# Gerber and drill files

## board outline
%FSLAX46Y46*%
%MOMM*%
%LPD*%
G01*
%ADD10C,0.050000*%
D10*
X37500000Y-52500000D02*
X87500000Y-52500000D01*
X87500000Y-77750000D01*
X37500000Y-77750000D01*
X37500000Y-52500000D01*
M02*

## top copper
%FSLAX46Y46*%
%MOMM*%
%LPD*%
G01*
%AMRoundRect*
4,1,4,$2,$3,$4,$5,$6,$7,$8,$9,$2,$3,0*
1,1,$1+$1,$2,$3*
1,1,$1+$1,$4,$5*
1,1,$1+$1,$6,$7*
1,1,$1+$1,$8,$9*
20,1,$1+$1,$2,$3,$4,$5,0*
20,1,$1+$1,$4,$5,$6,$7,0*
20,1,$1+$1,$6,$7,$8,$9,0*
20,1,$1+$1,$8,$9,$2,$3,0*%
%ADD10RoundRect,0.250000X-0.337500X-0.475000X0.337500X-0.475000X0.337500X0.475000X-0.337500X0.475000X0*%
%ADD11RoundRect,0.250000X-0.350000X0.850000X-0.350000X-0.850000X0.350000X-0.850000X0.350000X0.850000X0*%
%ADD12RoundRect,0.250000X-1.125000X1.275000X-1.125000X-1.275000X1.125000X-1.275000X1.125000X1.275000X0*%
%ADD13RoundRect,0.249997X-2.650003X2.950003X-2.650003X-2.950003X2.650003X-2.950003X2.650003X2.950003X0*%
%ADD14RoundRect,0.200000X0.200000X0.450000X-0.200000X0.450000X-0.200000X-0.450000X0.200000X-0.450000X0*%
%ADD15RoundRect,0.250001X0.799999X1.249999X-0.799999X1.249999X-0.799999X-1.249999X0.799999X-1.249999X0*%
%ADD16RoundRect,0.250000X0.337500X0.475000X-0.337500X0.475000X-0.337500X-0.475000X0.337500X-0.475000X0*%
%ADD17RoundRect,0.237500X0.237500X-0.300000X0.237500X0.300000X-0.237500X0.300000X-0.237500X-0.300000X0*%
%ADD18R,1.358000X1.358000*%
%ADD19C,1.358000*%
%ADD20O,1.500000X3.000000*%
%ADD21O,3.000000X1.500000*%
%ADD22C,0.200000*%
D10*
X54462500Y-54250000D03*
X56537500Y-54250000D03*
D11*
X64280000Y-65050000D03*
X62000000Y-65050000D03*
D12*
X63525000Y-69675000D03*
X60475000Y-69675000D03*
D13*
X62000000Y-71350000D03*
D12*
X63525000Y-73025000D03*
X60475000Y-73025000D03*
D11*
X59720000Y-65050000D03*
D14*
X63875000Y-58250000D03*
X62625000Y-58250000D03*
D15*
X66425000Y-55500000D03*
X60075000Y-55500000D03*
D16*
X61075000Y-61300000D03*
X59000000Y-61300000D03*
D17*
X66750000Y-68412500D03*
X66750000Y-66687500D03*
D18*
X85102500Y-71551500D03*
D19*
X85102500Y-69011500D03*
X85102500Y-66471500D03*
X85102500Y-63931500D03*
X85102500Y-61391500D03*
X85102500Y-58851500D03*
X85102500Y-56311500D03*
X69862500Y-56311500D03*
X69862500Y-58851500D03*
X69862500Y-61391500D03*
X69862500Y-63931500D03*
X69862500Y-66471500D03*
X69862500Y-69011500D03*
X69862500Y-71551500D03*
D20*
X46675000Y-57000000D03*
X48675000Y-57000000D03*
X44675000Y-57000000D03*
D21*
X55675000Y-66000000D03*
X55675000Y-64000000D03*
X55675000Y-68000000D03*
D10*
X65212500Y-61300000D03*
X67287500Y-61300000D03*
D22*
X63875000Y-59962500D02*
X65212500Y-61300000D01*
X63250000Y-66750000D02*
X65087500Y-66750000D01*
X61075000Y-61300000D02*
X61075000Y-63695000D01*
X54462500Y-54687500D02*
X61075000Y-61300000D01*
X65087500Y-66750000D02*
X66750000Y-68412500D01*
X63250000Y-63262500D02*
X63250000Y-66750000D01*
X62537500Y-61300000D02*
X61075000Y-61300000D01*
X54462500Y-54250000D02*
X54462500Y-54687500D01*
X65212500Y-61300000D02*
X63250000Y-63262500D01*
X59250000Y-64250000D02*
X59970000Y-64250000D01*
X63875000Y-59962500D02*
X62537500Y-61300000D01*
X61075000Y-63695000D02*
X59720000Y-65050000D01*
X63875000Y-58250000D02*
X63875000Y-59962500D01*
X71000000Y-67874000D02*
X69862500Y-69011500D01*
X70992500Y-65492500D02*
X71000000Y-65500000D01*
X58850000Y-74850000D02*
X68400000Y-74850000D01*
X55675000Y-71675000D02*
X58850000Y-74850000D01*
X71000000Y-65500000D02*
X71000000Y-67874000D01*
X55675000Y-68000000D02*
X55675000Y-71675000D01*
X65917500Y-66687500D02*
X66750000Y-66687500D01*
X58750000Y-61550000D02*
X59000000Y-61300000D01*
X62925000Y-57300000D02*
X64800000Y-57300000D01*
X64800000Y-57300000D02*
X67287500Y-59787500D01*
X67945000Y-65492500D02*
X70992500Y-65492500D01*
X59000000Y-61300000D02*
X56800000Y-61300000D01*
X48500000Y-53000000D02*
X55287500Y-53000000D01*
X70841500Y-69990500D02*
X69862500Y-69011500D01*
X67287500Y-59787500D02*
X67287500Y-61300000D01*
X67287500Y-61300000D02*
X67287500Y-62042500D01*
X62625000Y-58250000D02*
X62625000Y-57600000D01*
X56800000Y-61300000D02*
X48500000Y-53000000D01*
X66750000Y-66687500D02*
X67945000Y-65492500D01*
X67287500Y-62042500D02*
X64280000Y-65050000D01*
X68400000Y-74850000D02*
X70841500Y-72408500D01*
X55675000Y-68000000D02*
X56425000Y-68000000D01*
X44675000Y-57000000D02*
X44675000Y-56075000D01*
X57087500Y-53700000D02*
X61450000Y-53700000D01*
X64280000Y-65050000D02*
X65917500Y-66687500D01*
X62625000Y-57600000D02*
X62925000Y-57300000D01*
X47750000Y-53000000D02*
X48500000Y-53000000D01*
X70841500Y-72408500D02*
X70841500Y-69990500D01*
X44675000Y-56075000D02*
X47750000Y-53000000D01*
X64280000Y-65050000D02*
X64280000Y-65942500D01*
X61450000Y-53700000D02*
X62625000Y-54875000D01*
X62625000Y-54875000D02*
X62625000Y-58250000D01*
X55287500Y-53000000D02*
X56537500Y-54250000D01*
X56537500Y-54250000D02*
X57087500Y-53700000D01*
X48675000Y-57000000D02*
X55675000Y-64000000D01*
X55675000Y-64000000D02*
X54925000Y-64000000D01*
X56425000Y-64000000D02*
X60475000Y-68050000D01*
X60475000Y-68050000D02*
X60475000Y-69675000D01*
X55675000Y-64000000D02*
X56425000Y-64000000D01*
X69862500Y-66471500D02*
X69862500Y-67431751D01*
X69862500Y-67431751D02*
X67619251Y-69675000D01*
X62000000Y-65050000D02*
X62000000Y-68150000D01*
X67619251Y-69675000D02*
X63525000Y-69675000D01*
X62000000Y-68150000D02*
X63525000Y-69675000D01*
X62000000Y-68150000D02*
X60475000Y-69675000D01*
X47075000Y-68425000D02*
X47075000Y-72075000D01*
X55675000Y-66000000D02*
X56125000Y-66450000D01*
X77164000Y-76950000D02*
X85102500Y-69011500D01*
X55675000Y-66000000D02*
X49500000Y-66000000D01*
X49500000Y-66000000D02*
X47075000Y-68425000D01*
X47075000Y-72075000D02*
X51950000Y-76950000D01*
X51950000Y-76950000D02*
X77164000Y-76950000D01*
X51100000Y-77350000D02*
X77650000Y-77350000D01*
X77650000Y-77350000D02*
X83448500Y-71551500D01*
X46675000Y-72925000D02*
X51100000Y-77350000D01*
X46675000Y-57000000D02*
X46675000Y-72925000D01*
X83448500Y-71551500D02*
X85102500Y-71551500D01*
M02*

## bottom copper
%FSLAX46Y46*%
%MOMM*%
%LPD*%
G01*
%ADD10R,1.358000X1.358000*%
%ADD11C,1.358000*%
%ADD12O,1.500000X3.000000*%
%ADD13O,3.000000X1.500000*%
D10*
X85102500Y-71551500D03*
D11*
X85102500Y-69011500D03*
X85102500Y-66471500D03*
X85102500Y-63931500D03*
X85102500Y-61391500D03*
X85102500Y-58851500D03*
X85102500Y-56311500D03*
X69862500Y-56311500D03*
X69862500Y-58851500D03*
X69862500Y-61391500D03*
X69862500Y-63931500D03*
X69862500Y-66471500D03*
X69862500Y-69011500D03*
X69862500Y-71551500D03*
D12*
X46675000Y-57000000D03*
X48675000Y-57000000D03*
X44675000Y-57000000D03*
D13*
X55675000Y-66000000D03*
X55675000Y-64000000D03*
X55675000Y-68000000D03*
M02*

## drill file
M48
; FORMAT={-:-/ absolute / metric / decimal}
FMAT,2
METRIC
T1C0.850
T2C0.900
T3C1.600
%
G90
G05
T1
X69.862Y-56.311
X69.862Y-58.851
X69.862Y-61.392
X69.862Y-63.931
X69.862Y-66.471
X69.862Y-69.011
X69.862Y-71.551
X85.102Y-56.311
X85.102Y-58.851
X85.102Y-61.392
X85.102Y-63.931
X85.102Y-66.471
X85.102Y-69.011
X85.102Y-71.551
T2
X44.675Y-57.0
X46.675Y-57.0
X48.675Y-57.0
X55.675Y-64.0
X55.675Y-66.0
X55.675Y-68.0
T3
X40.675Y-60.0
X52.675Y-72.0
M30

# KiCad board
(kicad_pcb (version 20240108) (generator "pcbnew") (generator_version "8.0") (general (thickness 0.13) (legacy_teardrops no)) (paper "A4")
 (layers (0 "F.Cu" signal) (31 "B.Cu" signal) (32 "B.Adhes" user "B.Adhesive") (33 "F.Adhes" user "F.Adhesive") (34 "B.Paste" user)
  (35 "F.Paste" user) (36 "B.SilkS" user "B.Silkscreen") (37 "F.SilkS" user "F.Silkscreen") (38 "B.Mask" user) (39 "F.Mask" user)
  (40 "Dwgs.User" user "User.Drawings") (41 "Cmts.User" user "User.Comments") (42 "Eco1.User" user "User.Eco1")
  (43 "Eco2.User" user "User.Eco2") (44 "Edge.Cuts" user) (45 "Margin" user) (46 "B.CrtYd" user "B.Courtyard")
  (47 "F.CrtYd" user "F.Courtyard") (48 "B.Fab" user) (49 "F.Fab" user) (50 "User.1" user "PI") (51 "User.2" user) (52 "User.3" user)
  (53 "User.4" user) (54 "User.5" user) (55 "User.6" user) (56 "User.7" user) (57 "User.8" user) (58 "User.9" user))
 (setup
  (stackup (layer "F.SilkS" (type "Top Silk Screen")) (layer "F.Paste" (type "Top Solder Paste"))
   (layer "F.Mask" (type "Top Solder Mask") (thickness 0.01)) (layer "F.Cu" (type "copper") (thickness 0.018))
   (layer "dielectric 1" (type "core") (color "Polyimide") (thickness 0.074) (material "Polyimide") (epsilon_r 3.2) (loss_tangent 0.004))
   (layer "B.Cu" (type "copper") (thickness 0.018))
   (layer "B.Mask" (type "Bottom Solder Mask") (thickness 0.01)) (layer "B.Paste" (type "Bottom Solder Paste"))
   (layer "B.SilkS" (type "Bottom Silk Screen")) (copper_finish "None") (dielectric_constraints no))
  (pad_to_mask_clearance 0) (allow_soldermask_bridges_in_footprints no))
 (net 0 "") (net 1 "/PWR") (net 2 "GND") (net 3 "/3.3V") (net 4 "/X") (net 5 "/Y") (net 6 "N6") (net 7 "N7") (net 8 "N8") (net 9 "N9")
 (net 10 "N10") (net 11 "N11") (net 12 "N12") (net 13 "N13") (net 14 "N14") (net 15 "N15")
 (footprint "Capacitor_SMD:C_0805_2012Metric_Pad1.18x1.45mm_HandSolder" (layer "F.Cu") (at 55.5 54.25)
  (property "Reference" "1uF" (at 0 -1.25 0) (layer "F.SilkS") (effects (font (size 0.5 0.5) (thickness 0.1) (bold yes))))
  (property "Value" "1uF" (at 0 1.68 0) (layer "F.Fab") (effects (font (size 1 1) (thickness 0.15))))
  (pad "1" smd roundrect (at -1.0375 0) (size 1.175 1.45) (layers "F.Cu" "F.Paste" "F.Mask") (roundrect_rratio 0.212766) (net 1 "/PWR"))
  (pad "2" smd roundrect (at 1.0375 0) (size 1.175 1.45) (layers "F.Cu" "F.Paste" "F.Mask") (roundrect_rratio 0.212766) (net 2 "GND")))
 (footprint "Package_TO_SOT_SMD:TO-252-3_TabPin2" (layer "F.Cu") (at 62 70.09 -90)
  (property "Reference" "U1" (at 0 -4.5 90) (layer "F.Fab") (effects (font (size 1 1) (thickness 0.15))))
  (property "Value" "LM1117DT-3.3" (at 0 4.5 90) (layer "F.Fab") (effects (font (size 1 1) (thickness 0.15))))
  (pad "1" smd roundrect (at -5.04 -2.28 270) (size 2.2 1.2) (layers "F.Cu" "F.Paste" "F.Mask") (roundrect_rratio 0.208333) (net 2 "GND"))
  (pad "2" smd roundrect (at -5.04 0 270) (size 2.2 1.2) (layers "F.Cu" "F.Paste" "F.Mask") (roundrect_rratio 0.208333) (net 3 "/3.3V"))
  (pad "2" smd roundrect (at -0.415 -1.525 270) (size 3.05 2.75) (layers "F.Cu" "F.Paste") (roundrect_rratio 0.090909) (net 3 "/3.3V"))
  (pad "2" smd roundrect (at -0.415 1.525 270) (size 3.05 2.75) (layers "F.Cu" "F.Paste") (roundrect_rratio 0.090909) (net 3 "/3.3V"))
  (pad "2" smd roundrect (at 1.26 0 270) (size 6.4 5.8) (layers "F.Cu" "F.Mask") (roundrect_rratio 0.043103) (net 3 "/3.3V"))
  (pad "2" smd roundrect (at 2.935 -1.525 270) (size 3.05 2.75) (layers "F.Cu" "F.Paste") (roundrect_rratio 0.090909) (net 3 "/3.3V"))
  (pad "2" smd roundrect (at 2.935 1.525 270) (size 3.05 2.75) (layers "F.Cu" "F.Paste") (roundrect_rratio 0.090909) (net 3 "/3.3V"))
  (pad "3" smd roundrect (at -5.04 2.28 270) (size 2.2 1.2) (layers "F.Cu" "F.Paste" "F.Mask") (roundrect_rratio 0.208333) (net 1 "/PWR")))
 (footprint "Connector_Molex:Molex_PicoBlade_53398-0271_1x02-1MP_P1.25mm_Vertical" (layer "F.Cu") (at 63.25 57 180)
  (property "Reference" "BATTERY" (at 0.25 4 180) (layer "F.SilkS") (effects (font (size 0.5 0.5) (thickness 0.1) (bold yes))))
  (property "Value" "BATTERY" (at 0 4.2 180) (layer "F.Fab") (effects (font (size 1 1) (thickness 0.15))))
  (pad "1" smd roundrect (at -0.625 -1.25 180) (size 0.8 1.3) (layers "F.Cu" "F.Paste" "F.Mask") (roundrect_rratio 0.25) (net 1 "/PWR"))
  (pad "2" smd roundrect (at 0.625 -1.25 180) (size 0.8 1.3) (layers "F.Cu" "F.Paste" "F.Mask") (roundrect_rratio 0.25) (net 2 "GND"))
  (pad "MP" smd roundrect (at -3.175 1.5 180) (size 2.1 3) (layers "F.Cu" "F.Paste" "F.Mask") (roundrect_rratio 0.119048))
  (pad "MP" smd roundrect (at 3.175 1.5 180) (size 2.1 3) (layers "F.Cu" "F.Paste" "F.Mask") (roundrect_rratio 0.119048)))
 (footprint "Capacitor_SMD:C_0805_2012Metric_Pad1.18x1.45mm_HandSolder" (layer "F.Cu") (at 60.0375 61.3 180)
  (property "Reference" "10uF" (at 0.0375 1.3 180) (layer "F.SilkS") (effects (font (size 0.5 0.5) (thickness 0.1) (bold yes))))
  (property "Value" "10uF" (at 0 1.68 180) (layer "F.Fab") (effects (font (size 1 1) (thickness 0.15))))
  (pad "1" smd roundrect (at -1.0375 0 180) (size 1.175 1.45) (layers "F.Cu" "F.Paste" "F.Mask") (roundrect_rratio 0.212766) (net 1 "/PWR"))
  (pad "2" smd roundrect (at 1.0375 0 180) (size 1.175 1.45) (layers "F.Cu" "F.Paste" "F.Mask") (roundrect_rratio 0.212766) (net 2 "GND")))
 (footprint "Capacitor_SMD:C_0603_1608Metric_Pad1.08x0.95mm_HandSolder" (layer "F.Cu") (at 66.75 67.55 90)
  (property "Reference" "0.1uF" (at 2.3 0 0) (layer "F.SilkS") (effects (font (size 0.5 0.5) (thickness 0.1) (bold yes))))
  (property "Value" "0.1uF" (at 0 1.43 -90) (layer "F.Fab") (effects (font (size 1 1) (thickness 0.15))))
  (pad "1" smd roundrect (at -0.8625 0 90) (size 1.075 0.95) (layers "F.Cu" "F.Paste" "F.Mask") (roundrect_rratio 0.25) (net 1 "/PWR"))
  (pad "2" smd roundrect (at 0.8625 0 90) (size 1.075 0.95) (layers "F.Cu" "F.Paste" "F.Mask") (roundrect_rratio 0.25) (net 2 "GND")))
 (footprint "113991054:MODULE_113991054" (layer "F.Cu") (at 77.4825 63.995 180)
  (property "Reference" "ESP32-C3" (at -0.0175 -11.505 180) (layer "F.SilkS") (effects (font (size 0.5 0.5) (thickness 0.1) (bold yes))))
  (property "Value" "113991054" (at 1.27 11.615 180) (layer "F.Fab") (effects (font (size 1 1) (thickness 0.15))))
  (pad "1" thru_hole rect (at -7.62 -7.5565 180) (size 1.358 1.358) (drill 0.85) (layers "*.Cu" "*.Mask") (remove_unused_layers no)
   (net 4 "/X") (solder_mask_margin 0.102))
  (pad "2" thru_hole circle (at -7.62 -5.0165 180) (size 1.358 1.358) (drill 0.85) (layers "*.Cu" "*.Mask") (remove_unused_layers no)
   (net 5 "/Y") (solder_mask_margin 0.102))
  (pad "3" thru_hole circle (at -7.62 -2.4765 180) (size 1.358 1.358) (drill 0.85) (layers "*.Cu" "*.Mask") (remove_unused_layers no)
   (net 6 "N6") (solder_mask_margin 0.102))
  (pad "4" thru_hole circle (at -7.62 0.0635 180) (size 1.358 1.358) (drill 0.85) (layers "*.Cu" "*.Mask") (remove_unused_layers no)
   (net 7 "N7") (solder_mask_margin 0.102))
  (pad "5" thru_hole circle (at -7.62 2.6035 180) (size 1.358 1.358) (drill 0.85) (layers "*.Cu" "*.Mask") (remove_unused_layers no)
   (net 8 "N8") (solder_mask_margin 0.102))
  (pad "6" thru_hole circle (at -7.62 5.1435 180) (size 1.358 1.358) (drill 0.85) (layers "*.Cu" "*.Mask") (remove_unused_layers no)
   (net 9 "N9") (solder_mask_margin 0.102))
  (pad "7" thru_hole circle (at -7.62 7.6835 180) (size 1.358 1.358) (drill 0.85) (layers "*.Cu" "*.Mask") (remove_unused_layers no)
   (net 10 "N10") (solder_mask_margin 0.102))
  (pad "8" thru_hole circle (at 7.62 7.6835 180) (size 1.358 1.358) (drill 0.85) (layers "*.Cu" "*.Mask") (remove_unused_layers no)
   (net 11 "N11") (solder_mask_margin 0.102))
  (pad "9" thru_hole circle (at 7.62 5.1435 180) (size 1.358 1.358) (drill 0.85) (layers "*.Cu" "*.Mask") (remove_unused_layers no)
   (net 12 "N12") (solder_mask_margin 0.102))
  (pad "10" thru_hole circle (at 7.62 2.6035 180) (size 1.358 1.358) (drill 0.85) (layers "*.Cu" "*.Mask") (remove_unused_layers no)
   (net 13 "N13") (solder_mask_margin 0.102))
  (pad "11" thru_hole circle (at 7.62 0.0635 180) (size 1.358 1.358) (drill 0.85) (layers "*.Cu" "*.Mask") (remove_unused_layers no)
   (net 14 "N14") (solder_mask_margin 0.102))
  (pad "12" thru_hole circle (at 7.62 -2.4765 180) (size 1.358 1.358) (drill 0.85) (layers "*.Cu" "*.Mask") (remove_unused_layers no)
   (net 3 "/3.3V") (solder_mask_margin 0.102))
  (pad "13" thru_hole circle (at 7.62 -5.0165 180) (size 1.358 1.358) (drill 0.85) (layers "*.Cu" "*.Mask") (remove_unused_layers no)
   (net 2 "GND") (solder_mask_margin 0.102))
  (pad "14" thru_hole circle (at 7.62 -7.5565 180) (size 1.358 1.358) (drill 0.85) (layers "*.Cu" "*.Mask") (remove_unused_layers no)
   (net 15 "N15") (solder_mask_margin 0.102)))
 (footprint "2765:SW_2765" (layer "F.Cu") (at 46.675 66 90)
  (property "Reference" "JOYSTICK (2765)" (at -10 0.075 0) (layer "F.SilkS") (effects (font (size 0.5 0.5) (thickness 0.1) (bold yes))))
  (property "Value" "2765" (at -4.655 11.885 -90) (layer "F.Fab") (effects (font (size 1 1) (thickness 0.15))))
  (pad "" np_thru_hole circle (at -6 6 90) (size 1.6 1.6) (drill 1.6) (layers "*.Cu" "*.Mask"))
  (pad "" np_thru_hole circle (at 6 -6 90) (size 1.6 1.6) (drill 1.6) (layers "*.Cu" "*.Mask"))
  (pad "X" thru_hole oval (at 9 0 90) (size 3 1.5) (drill 0.9) (layers "*.Cu" "*.Mask") (remove_unused_layers no) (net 4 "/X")
   (solder_mask_margin 0.102))
  (pad "X+" thru_hole oval (at 9 2 90) (size 3 1.5) (drill 0.9) (layers "*.Cu" "*.Mask") (remove_unused_layers no) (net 3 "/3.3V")
   (solder_mask_margin 0.102))
  (pad "X-" thru_hole oval (at 9 -2 90) (size 3 1.5) (drill 0.9) (layers "*.Cu" "*.Mask") (remove_unused_layers no) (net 2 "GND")
   (solder_mask_margin 0.102))
  (pad "Y" thru_hole oval (at 0 9 90) (size 1.5 3) (drill 0.9) (layers "*.Cu" "*.Mask") (remove_unused_layers no) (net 5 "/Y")
   (solder_mask_margin 0.102))
  (pad "Y+" thru_hole oval (at 2 9 90) (size 1.5 3) (drill 0.9) (layers "*.Cu" "*.Mask") (remove_unused_layers no) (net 3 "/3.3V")
   (solder_mask_margin 0.102))
  (pad "Y-" thru_hole oval (at -2 9 90) (size 1.5 3) (drill 0.9) (layers "*.Cu" "*.Mask") (remove_unused_layers no) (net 2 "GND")
   (solder_mask_margin 0.102)))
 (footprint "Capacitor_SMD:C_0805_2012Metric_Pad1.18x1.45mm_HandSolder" (layer "F.Cu") (at 66.25 61.3)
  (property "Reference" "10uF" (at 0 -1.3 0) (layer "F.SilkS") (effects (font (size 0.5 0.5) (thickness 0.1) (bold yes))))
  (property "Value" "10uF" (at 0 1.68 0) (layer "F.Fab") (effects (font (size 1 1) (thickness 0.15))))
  (pad "1" smd roundrect (at -1.0375 0) (size 1.175 1.45) (layers "F.Cu" "F.Paste" "F.Mask") (roundrect_rratio 0.212766) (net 1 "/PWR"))
  (pad "2" smd roundrect (at 1.0375 0) (size 1.175 1.45) (layers "F.Cu" "F.Paste" "F.Mask") (roundrect_rratio 0.212766) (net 2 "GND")))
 (gr_rect (start 37.5 52.5) (end 87.5 77.75) (stroke (width 0.05) (type default)) (fill none) (layer "Edge.Cuts"))
 (segment (start 63.875 59.9625) (end 65.2125 61.3) (width 0.2) (layer "F.Cu") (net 1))
 (segment (start 63.25 66.75) (end 65.0875 66.75) (width 0.2) (layer "F.Cu") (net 1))
 (segment (start 61.075 61.3) (end 61.075 63.695) (width 0.2) (layer "F.Cu") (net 1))
 (segment (start 54.4625 54.6875) (end 61.075 61.3) (width 0.2) (layer "F.Cu") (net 1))
 (segment (start 65.0875 66.75) (end 66.75 68.4125) (width 0.2) (layer "F.Cu") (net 1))
 (segment (start 63.25 63.2625) (end 63.25 66.75) (width 0.2) (layer "F.Cu") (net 1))
 (segment (start 62.5375 61.3) (end 61.075 61.3) (width 0.2) (layer "F.Cu") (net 1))
 (segment (start 54.4625 54.25) (end 54.4625 54.6875) (width 0.2) (layer "F.Cu") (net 1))
 (segment (start 65.2125 61.3) (end 63.25 63.2625) (width 0.2) (layer "F.Cu") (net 1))
 (segment (start 59.25 64.25) (end 59.97 64.25) (width 0.2) (layer "F.Cu") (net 1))
 (segment (start 63.875 59.9625) (end 62.5375 61.3) (width 0.2) (layer "F.Cu") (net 1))
 (segment (start 61.075 63.695) (end 59.72 65.05) (width 0.2) (layer "F.Cu") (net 1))
 (segment (start 63.875 58.25) (end 63.875 59.9625) (width 0.2) (layer "F.Cu") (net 1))
 (segment (start 71 67.874) (end 69.8625 69.0115) (width 0.2) (layer "F.Cu") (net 2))
 (segment (start 70.9925 65.4925) (end 71 65.5) (width 0.2) (layer "F.Cu") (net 2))
 (segment (start 58.85 74.85) (end 68.4 74.85) (width 0.2) (layer "F.Cu") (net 2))
 (segment (start 55.675 71.675) (end 58.85 74.85) (width 0.2) (layer "F.Cu") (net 2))
 (segment (start 71 65.5) (end 71 67.874) (width 0.2) (layer "F.Cu") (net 2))
 (segment (start 55.675 68) (end 55.675 71.675) (width 0.2) (layer "F.Cu") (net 2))
 (segment (start 65.9175 66.6875) (end 66.75 66.6875) (width 0.2) (layer "F.Cu") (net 2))
 (segment (start 58.75 61.55) (end 59 61.3) (width 0.2) (layer "F.Cu") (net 2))
 (segment (start 62.925 57.3) (end 64.8 57.3) (width 0.2) (layer "F.Cu") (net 2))
 (segment (start 64.8 57.3) (end 67.2875 59.7875) (width 0.2) (layer "F.Cu") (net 2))
 (segment (start 67.945 65.4925) (end 70.9925 65.4925) (width 0.2) (layer "F.Cu") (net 2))
 (segment (start 59 61.3) (end 56.8 61.3) (width 0.2) (layer "F.Cu") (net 2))
 (segment (start 48.5 53) (end 55.2875 53) (width 0.2) (layer "F.Cu") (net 2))
 (segment (start 70.8415 69.9905) (end 69.8625 69.0115) (width 0.2) (layer "F.Cu") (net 2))
 (segment (start 67.2875 59.7875) (end 67.2875 61.3) (width 0.2) (layer "F.Cu") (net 2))
 (segment (start 67.2875 61.3) (end 67.2875 62.0425) (width 0.2) (layer "F.Cu") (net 2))
 (segment (start 62.625 58.25) (end 62.625 57.6) (width 0.2) (layer "F.Cu") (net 2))
 (segment (start 56.8 61.3) (end 48.5 53) (width 0.2) (layer "F.Cu") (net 2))
 (segment (start 66.75 66.6875) (end 67.945 65.4925) (width 0.2) (layer "F.Cu") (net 2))
 (segment (start 67.2875 62.0425) (end 64.28 65.05) (width 0.2) (layer "F.Cu") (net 2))
 (segment (start 68.4 74.85) (end 70.8415 72.4085) (width 0.2) (layer "F.Cu") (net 2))
 (segment (start 55.675 68) (end 56.425 68) (width 0.2) (layer "F.Cu") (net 2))
 (segment (start 44.675 57) (end 44.675 56.075) (width 0.2) (layer "F.Cu") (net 2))
 (segment (start 57.0875 53.7) (end 61.45 53.7) (width 0.2) (layer "F.Cu") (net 2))
 (segment (start 64.28 65.05) (end 65.9175 66.6875) (width 0.2) (layer "F.Cu") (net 2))
 (segment (start 62.625 57.6) (end 62.925 57.3) (width 0.2) (layer "F.Cu") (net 2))
 (segment (start 47.75 53) (end 48.5 53) (width 0.2) (layer "F.Cu") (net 2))
 (segment (start 70.8415 72.4085) (end 70.8415 69.9905) (width 0.2) (layer "F.Cu") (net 2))
 (segment (start 44.675 56.075) (end 47.75 53) (width 0.2) (layer "F.Cu") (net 2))
 (segment (start 64.28 65.05) (end 64.28 65.9425) (width 0.2) (layer "F.Cu") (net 2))
 (segment (start 61.45 53.7) (end 62.625 54.875) (width 0.2) (layer "F.Cu") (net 2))
 (segment (start 62.625 54.875) (end 62.625 58.25) (width 0.2) (layer "F.Cu") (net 2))
 (segment (start 55.2875 53) (end 56.5375 54.25) (width 0.2) (layer "F.Cu") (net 2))
 (segment (start 56.5375 54.25) (end 57.0875 53.7) (width 0.2) (layer "F.Cu") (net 2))
 (segment (start 48.675 57) (end 55.675 64) (width 0.2) (layer "F.Cu") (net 3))
 (segment (start 55.675 64) (end 54.925 64) (width 0.2) (layer "F.Cu") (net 3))
 (segment (start 56.425 64) (end 60.475 68.05) (width 0.2) (layer "F.Cu") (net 3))
 (segment (start 60.475 68.05) (end 60.475 69.675) (width 0.2) (layer "F.Cu") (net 3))
 (segment (start 55.675 64) (end 56.425 64) (width 0.2) (layer "F.Cu") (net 3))
 (segment (start 69.8625 66.4715) (end 69.8625 67.431751) (width 0.2) (layer "F.Cu") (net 3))
 (segment (start 69.8625 67.431751) (end 67.619251 69.675) (width 0.2) (layer "F.Cu") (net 3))
 (segment (start 62 65.05) (end 62 68.15) (width 0.2) (layer "F.Cu") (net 3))
 (segment (start 67.619251 69.675) (end 63.525 69.675) (width 0.2) (layer "F.Cu") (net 3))
 (segment (start 62 68.15) (end 63.525 69.675) (width 0.2) (layer "F.Cu") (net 3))
 (segment (start 62 68.15) (end 60.475 69.675) (width 0.2) (layer "F.Cu") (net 3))
 (segment (start 47.075 68.425) (end 47.075 72.075) (width 0.2) (layer "F.Cu") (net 5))
 (segment (start 55.675 66) (end 56.125 66.45) (width 0.2) (layer "F.Cu") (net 5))
 (segment (start 77.164 76.95) (end 85.1025 69.0115) (width 0.2) (layer "F.Cu") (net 5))
 (segment (start 55.675 66) (end 49.5 66) (width 0.2) (layer "F.Cu") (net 5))
 (segment (start 49.5 66) (end 47.075 68.425) (width 0.2) (layer "F.Cu") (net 5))
 (segment (start 47.075 72.075) (end 51.95 76.95) (width 0.2) (layer "F.Cu") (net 5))
 (segment (start 51.95 76.95) (end 77.164 76.95) (width 0.2) (layer "F.Cu") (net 5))
 (segment (start 51.1 77.35) (end 77.65 77.35) (width 0.2) (layer "F.Cu") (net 4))
 (segment (start 77.65 77.35) (end 83.4485 71.5515) (width 0.2) (layer "F.Cu") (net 4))
 (segment (start 46.675 72.925) (end 51.1 77.35) (width 0.2) (layer "F.Cu") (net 4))
 (segment (start 46.675 57) (end 46.675 72.925) (width 0.2) (layer "F.Cu") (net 4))
 (segment (start 83.4485 71.5515) (end 85.1025 71.5515) (width 0.2) (layer "F.Cu") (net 4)))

